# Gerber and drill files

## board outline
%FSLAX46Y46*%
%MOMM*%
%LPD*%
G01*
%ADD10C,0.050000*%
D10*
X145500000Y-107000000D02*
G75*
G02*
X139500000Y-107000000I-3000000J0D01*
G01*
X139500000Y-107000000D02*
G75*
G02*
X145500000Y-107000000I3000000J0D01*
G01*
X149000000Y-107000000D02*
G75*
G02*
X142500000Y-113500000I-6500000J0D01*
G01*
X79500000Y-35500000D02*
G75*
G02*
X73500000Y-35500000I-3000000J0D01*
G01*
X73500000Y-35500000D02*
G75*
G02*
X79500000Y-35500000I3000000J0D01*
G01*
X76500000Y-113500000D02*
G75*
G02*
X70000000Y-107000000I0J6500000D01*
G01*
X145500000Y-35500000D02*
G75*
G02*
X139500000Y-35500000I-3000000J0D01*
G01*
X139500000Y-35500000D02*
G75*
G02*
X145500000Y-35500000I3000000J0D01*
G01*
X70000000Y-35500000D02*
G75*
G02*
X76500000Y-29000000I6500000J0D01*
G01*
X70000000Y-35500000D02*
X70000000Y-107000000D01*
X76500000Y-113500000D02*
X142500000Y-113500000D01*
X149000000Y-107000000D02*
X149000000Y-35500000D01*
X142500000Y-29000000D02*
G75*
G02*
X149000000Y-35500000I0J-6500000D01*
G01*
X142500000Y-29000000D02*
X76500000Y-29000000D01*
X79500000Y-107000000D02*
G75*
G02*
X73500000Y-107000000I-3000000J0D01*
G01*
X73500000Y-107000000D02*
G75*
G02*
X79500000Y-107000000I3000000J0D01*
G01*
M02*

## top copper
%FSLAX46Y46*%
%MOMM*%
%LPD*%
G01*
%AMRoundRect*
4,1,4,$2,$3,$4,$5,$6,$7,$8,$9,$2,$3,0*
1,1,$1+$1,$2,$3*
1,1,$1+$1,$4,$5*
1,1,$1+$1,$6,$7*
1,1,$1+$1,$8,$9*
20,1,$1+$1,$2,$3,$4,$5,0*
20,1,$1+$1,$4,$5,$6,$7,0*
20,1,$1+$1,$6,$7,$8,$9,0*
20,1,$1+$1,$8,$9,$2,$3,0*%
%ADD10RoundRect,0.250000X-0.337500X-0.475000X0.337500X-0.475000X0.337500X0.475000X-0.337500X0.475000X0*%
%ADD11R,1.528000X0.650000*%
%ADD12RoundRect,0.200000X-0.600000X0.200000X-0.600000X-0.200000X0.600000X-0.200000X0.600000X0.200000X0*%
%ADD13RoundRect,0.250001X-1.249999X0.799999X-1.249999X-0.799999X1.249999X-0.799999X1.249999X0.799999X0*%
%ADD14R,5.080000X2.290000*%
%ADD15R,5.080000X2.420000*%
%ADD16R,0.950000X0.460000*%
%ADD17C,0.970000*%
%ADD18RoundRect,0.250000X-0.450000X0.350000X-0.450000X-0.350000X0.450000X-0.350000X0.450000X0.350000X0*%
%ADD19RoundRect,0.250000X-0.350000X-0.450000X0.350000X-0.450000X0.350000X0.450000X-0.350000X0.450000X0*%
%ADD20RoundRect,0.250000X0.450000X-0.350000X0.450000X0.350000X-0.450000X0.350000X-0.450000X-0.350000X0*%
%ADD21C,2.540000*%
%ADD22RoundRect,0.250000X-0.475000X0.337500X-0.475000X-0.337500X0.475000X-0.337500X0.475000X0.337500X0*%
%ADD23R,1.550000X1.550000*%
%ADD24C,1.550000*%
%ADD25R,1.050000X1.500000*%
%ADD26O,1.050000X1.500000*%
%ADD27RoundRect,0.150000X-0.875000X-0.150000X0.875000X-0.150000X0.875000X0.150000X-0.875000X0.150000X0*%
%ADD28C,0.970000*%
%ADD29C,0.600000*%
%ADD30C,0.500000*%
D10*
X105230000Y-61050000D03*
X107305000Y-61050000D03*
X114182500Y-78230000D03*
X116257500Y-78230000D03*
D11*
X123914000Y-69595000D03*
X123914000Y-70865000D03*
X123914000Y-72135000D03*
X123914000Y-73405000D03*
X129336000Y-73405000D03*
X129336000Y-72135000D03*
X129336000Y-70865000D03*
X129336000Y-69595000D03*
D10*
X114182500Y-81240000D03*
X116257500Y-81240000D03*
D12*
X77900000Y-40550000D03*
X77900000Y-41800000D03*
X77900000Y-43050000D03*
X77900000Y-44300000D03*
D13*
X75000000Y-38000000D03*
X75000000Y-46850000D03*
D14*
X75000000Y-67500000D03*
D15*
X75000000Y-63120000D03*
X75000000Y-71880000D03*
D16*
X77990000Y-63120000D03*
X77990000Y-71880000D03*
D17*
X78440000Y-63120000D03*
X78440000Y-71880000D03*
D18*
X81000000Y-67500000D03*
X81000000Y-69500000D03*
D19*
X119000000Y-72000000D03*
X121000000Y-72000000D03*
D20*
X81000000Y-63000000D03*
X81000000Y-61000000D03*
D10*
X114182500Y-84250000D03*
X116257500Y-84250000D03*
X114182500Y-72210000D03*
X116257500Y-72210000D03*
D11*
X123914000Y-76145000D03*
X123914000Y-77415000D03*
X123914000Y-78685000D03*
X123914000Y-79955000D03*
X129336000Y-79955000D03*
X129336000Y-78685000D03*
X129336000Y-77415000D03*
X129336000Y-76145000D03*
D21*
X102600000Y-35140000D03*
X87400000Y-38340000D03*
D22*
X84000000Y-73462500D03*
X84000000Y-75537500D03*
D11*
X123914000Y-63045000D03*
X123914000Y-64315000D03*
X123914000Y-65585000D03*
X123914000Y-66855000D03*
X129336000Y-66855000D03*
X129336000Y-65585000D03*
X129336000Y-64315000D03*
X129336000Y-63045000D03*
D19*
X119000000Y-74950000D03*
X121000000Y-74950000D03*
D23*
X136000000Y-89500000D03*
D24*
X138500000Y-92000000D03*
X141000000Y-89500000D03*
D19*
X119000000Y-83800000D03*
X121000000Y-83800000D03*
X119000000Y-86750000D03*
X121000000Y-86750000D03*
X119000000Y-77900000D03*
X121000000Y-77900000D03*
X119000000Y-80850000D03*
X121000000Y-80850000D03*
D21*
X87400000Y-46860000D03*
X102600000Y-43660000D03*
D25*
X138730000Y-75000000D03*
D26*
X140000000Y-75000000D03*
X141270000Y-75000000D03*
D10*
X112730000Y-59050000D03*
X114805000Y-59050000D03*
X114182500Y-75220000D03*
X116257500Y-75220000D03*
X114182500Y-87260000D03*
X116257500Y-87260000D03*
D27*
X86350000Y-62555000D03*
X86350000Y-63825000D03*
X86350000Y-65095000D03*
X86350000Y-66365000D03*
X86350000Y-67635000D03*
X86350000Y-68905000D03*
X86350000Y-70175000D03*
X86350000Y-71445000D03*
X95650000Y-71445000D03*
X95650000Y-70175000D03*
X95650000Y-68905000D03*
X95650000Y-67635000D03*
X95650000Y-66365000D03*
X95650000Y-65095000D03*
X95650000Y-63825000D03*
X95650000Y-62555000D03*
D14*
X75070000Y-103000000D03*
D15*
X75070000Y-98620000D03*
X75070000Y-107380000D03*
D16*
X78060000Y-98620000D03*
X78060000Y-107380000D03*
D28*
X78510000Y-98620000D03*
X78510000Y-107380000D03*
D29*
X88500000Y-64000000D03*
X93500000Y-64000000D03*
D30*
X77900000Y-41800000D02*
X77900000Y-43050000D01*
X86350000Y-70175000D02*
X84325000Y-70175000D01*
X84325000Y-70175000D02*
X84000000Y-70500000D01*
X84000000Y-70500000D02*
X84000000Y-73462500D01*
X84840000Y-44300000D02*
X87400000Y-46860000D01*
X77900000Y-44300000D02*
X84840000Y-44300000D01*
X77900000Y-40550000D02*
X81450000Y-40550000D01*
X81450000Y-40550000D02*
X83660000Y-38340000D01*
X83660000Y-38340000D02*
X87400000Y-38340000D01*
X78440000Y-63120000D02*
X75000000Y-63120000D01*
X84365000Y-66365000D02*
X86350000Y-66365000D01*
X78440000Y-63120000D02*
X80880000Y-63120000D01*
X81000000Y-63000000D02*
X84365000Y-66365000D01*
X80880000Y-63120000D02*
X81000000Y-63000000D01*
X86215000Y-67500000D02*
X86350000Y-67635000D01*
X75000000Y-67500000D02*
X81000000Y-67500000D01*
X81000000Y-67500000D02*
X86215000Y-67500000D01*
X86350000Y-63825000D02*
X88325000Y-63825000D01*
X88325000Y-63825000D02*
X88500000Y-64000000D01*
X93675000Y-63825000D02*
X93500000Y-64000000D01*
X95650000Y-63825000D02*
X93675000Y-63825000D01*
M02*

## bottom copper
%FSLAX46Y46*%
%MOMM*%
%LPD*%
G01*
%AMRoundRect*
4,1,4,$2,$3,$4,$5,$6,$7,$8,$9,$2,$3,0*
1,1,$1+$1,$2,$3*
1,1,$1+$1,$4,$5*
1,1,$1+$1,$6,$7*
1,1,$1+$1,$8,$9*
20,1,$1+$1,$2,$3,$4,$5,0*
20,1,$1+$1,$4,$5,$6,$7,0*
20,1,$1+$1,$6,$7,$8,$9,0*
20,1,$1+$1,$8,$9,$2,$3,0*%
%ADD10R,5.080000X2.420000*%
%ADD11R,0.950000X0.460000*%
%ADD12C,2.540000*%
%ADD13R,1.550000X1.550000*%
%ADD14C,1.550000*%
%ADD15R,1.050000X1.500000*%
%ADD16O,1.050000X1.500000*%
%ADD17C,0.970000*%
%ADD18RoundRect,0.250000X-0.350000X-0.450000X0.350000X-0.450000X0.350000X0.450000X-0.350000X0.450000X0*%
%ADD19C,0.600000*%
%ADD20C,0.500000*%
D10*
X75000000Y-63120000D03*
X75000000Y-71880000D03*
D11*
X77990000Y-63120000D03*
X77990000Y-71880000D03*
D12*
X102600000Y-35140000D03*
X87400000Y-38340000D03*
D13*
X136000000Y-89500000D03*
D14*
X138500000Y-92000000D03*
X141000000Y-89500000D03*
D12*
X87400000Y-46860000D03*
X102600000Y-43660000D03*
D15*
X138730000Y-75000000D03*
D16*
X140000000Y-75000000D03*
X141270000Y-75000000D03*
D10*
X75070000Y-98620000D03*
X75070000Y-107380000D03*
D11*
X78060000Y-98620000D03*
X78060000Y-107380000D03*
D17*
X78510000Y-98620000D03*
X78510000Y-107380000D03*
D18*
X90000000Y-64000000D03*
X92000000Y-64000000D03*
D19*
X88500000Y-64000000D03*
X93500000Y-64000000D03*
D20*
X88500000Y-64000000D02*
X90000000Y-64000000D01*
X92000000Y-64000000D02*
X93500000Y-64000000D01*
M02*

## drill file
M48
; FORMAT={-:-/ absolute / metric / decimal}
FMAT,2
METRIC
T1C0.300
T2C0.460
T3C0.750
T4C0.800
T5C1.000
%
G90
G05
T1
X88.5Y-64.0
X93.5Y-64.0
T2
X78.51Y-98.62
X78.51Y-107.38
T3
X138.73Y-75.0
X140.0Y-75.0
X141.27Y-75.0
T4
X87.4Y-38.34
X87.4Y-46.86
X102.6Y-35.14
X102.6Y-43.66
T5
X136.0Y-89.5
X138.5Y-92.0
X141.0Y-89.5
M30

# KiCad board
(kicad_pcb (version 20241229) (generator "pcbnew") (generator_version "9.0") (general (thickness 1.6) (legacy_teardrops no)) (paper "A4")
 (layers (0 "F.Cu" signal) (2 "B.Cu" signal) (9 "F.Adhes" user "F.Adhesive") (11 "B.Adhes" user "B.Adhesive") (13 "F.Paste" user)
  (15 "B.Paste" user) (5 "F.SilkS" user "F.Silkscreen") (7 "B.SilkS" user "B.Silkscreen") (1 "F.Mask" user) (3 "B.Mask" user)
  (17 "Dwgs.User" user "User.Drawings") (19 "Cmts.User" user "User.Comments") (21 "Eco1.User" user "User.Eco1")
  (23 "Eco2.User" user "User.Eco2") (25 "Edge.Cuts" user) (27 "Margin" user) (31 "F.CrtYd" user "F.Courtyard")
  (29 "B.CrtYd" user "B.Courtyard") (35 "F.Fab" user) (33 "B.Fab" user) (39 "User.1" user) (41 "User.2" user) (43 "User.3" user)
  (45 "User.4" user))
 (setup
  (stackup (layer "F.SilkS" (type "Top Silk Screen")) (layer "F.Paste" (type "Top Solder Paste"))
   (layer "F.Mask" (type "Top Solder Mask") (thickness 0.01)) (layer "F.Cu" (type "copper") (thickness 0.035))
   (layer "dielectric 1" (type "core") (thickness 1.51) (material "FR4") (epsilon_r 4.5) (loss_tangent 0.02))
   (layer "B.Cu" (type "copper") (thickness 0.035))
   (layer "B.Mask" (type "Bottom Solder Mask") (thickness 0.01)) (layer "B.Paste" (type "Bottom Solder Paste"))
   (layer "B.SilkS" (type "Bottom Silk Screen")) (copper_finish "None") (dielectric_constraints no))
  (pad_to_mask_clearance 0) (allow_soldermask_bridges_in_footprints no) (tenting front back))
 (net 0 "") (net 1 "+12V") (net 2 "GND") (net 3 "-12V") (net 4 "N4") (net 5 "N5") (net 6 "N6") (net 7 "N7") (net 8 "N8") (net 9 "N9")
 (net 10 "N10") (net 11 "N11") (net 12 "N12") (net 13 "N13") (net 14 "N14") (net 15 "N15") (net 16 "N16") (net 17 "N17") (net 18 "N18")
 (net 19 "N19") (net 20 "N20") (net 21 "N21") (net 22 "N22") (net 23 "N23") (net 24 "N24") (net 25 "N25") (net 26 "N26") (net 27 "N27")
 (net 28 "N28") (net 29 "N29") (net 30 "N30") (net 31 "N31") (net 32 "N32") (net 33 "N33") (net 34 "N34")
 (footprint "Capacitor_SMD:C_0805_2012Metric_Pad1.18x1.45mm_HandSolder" (layer "F.Cu") (at 106.2675 61.05)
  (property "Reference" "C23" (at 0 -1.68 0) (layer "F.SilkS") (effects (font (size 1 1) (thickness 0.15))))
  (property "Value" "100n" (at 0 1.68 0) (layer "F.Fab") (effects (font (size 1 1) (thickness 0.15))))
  (pad "1" smd roundrect (at -1.0375 0) (size 1.175 1.45) (layers "F.Cu" "F.Mask" "F.Paste") (roundrect_rratio 0.212766) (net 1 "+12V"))
  (pad "2" smd roundrect (at 1.0375 0) (size 1.175 1.45) (layers "F.Cu" "F.Mask" "F.Paste") (roundrect_rratio 0.212766) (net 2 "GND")))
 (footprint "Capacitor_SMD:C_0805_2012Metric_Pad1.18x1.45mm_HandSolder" (layer "F.Cu") (at 115.22 78.23)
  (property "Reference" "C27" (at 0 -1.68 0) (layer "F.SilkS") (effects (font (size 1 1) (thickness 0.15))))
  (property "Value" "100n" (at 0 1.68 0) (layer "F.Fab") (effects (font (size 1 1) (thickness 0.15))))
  (pad "1" smd roundrect (at -1.0375 0) (size 1.175 1.45) (layers "F.Cu" "F.Mask" "F.Paste") (roundrect_rratio 0.212766) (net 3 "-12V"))
  (pad "2" smd roundrect (at 1.0375 0) (size 1.175 1.45) (layers "F.Cu" "F.Mask" "F.Paste") (roundrect_rratio 0.212766) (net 2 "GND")))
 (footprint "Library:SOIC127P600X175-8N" (layer "F.Cu") (at 126.625 71.5)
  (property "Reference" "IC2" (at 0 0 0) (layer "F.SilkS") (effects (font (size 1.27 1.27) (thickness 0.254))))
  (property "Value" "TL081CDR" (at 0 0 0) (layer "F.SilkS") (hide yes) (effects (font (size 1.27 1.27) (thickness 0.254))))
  (pad "1" smd rect (at -2.711 -1.905 90) (size 0.65 1.528) (layers "F.Cu" "F.Mask" "F.Paste") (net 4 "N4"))
  (pad "2" smd rect (at -2.711 -0.635 90) (size 0.65 1.528) (layers "F.Cu" "F.Mask" "F.Paste") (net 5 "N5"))
  (pad "3" smd rect (at -2.711 0.635 90) (size 0.65 1.528) (layers "F.Cu" "F.Mask" "F.Paste") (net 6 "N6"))
  (pad "4" smd rect (at -2.711 1.905 90) (size 0.65 1.528) (layers "F.Cu" "F.Mask" "F.Paste") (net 3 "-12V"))
  (pad "5" smd rect (at 2.711 1.905 90) (size 0.65 1.528) (layers "F.Cu" "F.Mask" "F.Paste") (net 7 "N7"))
  (pad "6" smd rect (at 2.711 0.635 90) (size 0.65 1.528) (layers "F.Cu" "F.Mask" "F.Paste") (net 5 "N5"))
  (pad "7" smd rect (at 2.711 -0.635 90) (size 0.65 1.528) (layers "F.Cu" "F.Mask" "F.Paste") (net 1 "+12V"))
  (pad "8" smd rect (at 2.711 -1.905 90) (size 0.65 1.528) (layers "F.Cu" "F.Mask" "F.Paste") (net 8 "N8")))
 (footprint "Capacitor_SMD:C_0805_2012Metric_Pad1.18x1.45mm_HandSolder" (layer "F.Cu") (at 115.22 81.24)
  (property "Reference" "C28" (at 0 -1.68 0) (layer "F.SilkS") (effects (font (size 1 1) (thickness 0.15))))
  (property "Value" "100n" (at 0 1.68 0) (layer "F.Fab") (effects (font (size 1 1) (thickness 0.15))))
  (pad "1" smd roundrect (at -1.0375 0) (size 1.175 1.45) (layers "F.Cu" "F.Mask" "F.Paste") (roundrect_rratio 0.212766) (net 1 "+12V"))
  (pad "2" smd roundrect (at 1.0375 0) (size 1.175 1.45) (layers "F.Cu" "F.Mask" "F.Paste") (roundrect_rratio 0.212766) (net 2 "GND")))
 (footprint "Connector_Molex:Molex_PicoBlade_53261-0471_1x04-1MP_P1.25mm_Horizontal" (layer "F.Cu") (at 75.5 42.425 -90)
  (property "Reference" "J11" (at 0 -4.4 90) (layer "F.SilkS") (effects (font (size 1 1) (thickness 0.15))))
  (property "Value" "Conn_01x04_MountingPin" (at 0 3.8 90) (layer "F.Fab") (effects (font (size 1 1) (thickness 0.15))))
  (pad "1" smd roundrect (at -1.875 -2.4 270) (size 0.8 1.6) (layers "F.Cu" "F.Mask" "F.Paste") (roundrect_rratio 0.25) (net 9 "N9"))
  (pad "2" smd roundrect (at -0.625 -2.4 270) (size 0.8 1.6) (layers "F.Cu" "F.Mask" "F.Paste") (roundrect_rratio 0.25) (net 2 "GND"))
  (pad "3" smd roundrect (at 0.625 -2.4 270) (size 0.8 1.6) (layers "F.Cu" "F.Mask" "F.Paste") (roundrect_rratio 0.25) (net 2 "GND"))
  (pad "4" smd roundrect (at 1.875 -2.4 270) (size 0.8 1.6) (layers "F.Cu" "F.Mask" "F.Paste") (roundrect_rratio 0.25) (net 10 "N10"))
  (pad "MP" smd roundrect (at -4.425 0.5 270) (size 2.1 3) (layers "F.Cu" "F.Mask" "F.Paste") (roundrect_rratio 0.119048) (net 2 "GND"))
  (pad "MP" smd roundrect (at 4.425 0.5 270) (size 2.1 3) (layers "F.Cu" "F.Mask" "F.Paste") (roundrect_rratio 0.119048) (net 2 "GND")))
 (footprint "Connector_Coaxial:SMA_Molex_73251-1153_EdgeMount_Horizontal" (layer "F.Cu") (at 76.72 67.5)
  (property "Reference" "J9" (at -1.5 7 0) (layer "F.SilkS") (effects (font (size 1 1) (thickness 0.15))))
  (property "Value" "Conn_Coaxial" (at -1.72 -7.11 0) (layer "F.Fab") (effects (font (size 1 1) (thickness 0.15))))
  (pad "1" smd rect (at -1.72 0) (size 5.08 2.29) (layers "F.Cu" "F.Mask" "F.Paste") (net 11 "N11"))
  (pad "2" smd rect (at -1.72 -4.38) (size 5.08 2.42) (layers "F.Cu" "F.Mask" "F.Paste") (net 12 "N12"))
  (pad "2" smd rect (at -1.72 -4.38) (size 5.08 2.42) (layers "B.Cu" "B.Mask" "B.Paste") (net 12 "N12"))
  (pad "2" smd rect (at -1.72 4.38) (size 5.08 2.42) (layers "F.Cu" "F.Mask" "F.Paste") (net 12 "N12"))
  (pad "2" smd rect (at -1.72 4.38) (size 5.08 2.42) (layers "B.Cu" "B.Mask" "B.Paste") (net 12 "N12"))
  (pad "2" smd rect (at 1.27 -4.38) (size 0.95 0.46) (layers "F.Cu") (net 12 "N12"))
  (pad "2" smd rect (at 1.27 -4.38) (size 0.95 0.46) (layers "B.Cu") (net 12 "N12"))
  (pad "2" smd rect (at 1.27 4.38) (size 0.95 0.46) (layers "F.Cu") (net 12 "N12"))
  (pad "2" smd rect (at 1.27 4.38) (size 0.95 0.46) (layers "B.Cu") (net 12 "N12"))
  (pad "2" smd circle (at 1.72 -4.38) (size 0.97 0.97) (layers "F.Cu" "F.Mask" "F.Paste") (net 12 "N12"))
  (pad "2" smd circle (at 1.72 4.38) (size 0.97 0.97) (layers "F.Cu" "F.Mask" "F.Paste") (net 12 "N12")))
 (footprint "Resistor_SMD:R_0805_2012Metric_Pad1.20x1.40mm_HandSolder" (layer "F.Cu") (at 81 68.5 -90)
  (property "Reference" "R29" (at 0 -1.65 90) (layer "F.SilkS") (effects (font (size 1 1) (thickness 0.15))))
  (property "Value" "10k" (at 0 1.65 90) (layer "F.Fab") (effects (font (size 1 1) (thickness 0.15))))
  (pad "1" smd roundrect (at -1 0 270) (size 1.2 1.4) (layers "F.Cu" "F.Mask" "F.Paste") (roundrect_rratio 0.208333) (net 11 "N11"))
  (pad "2" smd roundrect (at 1 0 270) (size 1.2 1.4) (layers "F.Cu" "F.Mask" "F.Paste") (roundrect_rratio 0.208333) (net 2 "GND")))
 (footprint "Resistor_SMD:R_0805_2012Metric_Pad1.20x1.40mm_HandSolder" (layer "F.Cu") (at 120 72)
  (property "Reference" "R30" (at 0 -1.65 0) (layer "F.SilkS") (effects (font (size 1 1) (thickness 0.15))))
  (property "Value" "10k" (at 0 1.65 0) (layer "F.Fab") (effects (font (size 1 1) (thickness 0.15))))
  (pad "1" smd roundrect (at -1 0) (size 1.2 1.4) (layers "F.Cu" "F.Mask" "F.Paste") (roundrect_rratio 0.208333) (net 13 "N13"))
  (pad "2" smd roundrect (at 1 0) (size 1.2 1.4) (layers "F.Cu" "F.Mask" "F.Paste") (roundrect_rratio 0.208333) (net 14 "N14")))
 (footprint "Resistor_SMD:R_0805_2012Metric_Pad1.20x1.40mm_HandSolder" (layer "F.Cu") (at 81 62 90)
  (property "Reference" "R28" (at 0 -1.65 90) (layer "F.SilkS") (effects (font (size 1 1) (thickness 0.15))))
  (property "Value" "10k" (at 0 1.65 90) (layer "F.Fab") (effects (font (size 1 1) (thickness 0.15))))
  (pad "1" smd roundrect (at -1 0 90) (size 1.2 1.4) (layers "F.Cu" "F.Mask" "F.Paste") (roundrect_rratio 0.208333) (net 12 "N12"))
  (pad "2" smd roundrect (at 1 0 90) (size 1.2 1.4) (layers "F.Cu" "F.Mask" "F.Paste") (roundrect_rratio 0.208333) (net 2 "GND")))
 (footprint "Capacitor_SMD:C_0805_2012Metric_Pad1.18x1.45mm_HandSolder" (layer "F.Cu") (at 115.22 84.25)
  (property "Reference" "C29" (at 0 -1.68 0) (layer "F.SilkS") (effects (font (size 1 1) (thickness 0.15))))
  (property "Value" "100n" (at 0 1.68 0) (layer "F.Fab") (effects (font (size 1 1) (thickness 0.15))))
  (pad "1" smd roundrect (at -1.0375 0) (size 1.175 1.45) (layers "F.Cu" "F.Mask" "F.Paste") (roundrect_rratio 0.212766) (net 3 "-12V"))
  (pad "2" smd roundrect (at 1.0375 0) (size 1.175 1.45) (layers "F.Cu" "F.Mask" "F.Paste") (roundrect_rratio 0.212766) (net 2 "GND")))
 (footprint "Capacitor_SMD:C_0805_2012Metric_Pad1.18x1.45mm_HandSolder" (layer "F.Cu") (at 115.22 72.21)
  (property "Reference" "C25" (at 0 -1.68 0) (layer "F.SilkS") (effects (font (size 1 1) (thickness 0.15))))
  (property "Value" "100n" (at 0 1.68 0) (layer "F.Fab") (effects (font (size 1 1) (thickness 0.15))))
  (pad "1" smd roundrect (at -1.0375 0) (size 1.175 1.45) (layers "F.Cu" "F.Mask" "F.Paste") (roundrect_rratio 0.212766) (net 3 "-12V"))
  (pad "2" smd roundrect (at 1.0375 0) (size 1.175 1.45) (layers "F.Cu" "F.Mask" "F.Paste") (roundrect_rratio 0.212766) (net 2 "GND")))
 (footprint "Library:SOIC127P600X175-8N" (layer "F.Cu") (at 126.625 78.05)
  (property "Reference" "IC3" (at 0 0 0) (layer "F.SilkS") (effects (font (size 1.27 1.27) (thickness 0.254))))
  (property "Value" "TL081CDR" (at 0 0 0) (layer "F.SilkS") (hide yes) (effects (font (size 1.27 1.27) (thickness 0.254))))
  (pad "1" smd rect (at -2.711 -1.905 90) (size 0.65 1.528) (layers "F.Cu" "F.Mask" "F.Paste") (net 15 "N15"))
  (pad "2" smd rect (at -2.711 -0.635 90) (size 0.65 1.528) (layers "F.Cu" "F.Mask" "F.Paste") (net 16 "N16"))
  (pad "3" smd rect (at -2.711 0.635 90) (size 0.65 1.528) (layers "F.Cu" "F.Mask" "F.Paste") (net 14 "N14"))
  (pad "4" smd rect (at -2.711 1.905 90) (size 0.65 1.528) (layers "F.Cu" "F.Mask" "F.Paste") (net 3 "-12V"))
  (pad "5" smd rect (at 2.711 1.905 90) (size 0.65 1.528) (layers "F.Cu" "F.Mask" "F.Paste") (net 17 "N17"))
  (pad "6" smd rect (at 2.711 0.635 90) (size 0.65 1.528) (layers "F.Cu" "F.Mask" "F.Paste") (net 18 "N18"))
  (pad "7" smd rect (at 2.711 -0.635 90) (size 0.65 1.528) (layers "F.Cu" "F.Mask" "F.Paste") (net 1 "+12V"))
  (pad "8" smd rect (at 2.711 -1.905 90) (size 0.65 1.528) (layers "F.Cu" "F.Mask" "F.Paste") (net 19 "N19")))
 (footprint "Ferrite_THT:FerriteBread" (layer "F.Cu") (at 95.1 32.64 180)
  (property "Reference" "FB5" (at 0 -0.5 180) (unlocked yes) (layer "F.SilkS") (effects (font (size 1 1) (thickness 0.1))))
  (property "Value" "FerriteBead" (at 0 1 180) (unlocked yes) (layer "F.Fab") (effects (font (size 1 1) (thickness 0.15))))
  (pad "1" thru_hole circle (at -7.5 -2.5 180) (size 2.54 2.54) (drill 0.8) (layers "*.Cu" "*.Mask") (remove_unused_layers no)
   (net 1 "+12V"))
  (pad "2" thru_hole circle (at 7.7 -5.7 180) (size 2.54 2.54) (drill 0.8) (layers "*.Cu" "*.Mask") (remove_unused_layers no) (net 9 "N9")))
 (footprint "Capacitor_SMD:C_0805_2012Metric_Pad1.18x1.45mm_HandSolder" (layer "F.Cu") (at 84 74.5 -90)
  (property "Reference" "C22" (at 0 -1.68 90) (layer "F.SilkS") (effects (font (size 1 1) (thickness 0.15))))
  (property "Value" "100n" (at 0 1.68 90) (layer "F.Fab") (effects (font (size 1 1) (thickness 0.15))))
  (pad "1" smd roundrect (at -1.0375 0 270) (size 1.175 1.45) (layers "F.Cu" "F.Mask" "F.Paste") (roundrect_rratio 0.212766) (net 3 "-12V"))
  (pad "2" smd roundrect (at 1.0375 0 270) (size 1.175 1.45) (layers "F.Cu" "F.Mask" "F.Paste") (roundrect_rratio 0.212766) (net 2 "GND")))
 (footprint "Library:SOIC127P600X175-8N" (layer "F.Cu") (at 126.625 64.95)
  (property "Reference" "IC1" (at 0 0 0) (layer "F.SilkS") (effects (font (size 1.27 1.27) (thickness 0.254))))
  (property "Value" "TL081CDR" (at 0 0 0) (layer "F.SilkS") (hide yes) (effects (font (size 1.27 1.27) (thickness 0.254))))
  (pad "1" smd rect (at -2.711 -1.905 90) (size 0.65 1.528) (layers "F.Cu" "F.Mask" "F.Paste") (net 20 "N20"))
  (pad "2" smd rect (at -2.711 -0.635 90) (size 0.65 1.528) (layers "F.Cu" "F.Mask" "F.Paste") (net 13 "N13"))
  (pad "3" smd rect (at -2.711 0.635 90) (size 0.65 1.528) (layers "F.Cu" "F.Mask" "F.Paste") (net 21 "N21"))
  (pad "4" smd rect (at -2.711 1.905 90) (size 0.65 1.528) (layers "F.Cu" "F.Mask" "F.Paste") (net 3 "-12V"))
  (pad "5" smd rect (at 2.711 1.905 90) (size 0.65 1.528) (layers "F.Cu" "F.Mask" "F.Paste") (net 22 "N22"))
  (pad "6" smd rect (at 2.711 0.635 90) (size 0.65 1.528) (layers "F.Cu" "F.Mask" "F.Paste") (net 13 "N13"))
  (pad "7" smd rect (at 2.711 -0.635 90) (size 0.65 1.528) (layers "F.Cu" "F.Mask" "F.Paste") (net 1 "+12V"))
  (pad "8" smd rect (at 2.711 -1.905 90) (size 0.65 1.528) (layers "F.Cu" "F.Mask" "F.Paste") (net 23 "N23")))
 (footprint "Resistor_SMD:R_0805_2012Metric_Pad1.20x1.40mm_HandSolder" (layer "F.Cu") (at 120 74.95)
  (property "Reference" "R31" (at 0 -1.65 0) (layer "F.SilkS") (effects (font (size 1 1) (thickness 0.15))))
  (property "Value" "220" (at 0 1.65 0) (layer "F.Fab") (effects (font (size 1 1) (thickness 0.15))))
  (pad "1" smd roundrect (at -1 0) (size 1.2 1.4) (layers "F.Cu" "F.Mask" "F.Paste") (roundrect_rratio 0.208333) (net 1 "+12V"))
  (pad "2" smd roundrect (at 1 0) (size 1.2 1.4) (layers "F.Cu" "F.Mask" "F.Paste") (roundrect_rratio 0.208333) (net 6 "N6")))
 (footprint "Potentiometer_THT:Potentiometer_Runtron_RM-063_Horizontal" (layer "F.Cu") (at 136 89.5)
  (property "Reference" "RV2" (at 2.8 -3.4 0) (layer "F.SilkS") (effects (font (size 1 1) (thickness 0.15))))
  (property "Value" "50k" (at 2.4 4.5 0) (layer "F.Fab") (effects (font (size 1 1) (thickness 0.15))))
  (pad "1" thru_hole rect (at 0 0) (size 1.55 1.55) (drill 1) (layers "*.Cu" "*.Mask") (remove_unused_layers no) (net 6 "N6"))
  (pad "2" thru_hole circle (at 2.5 2.5) (size 1.55 1.55) (drill 1) (layers "*.Cu" "*.Mask") (remove_unused_layers no) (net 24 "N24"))
  (pad "3" thru_hole circle (at 5 0) (size 1.55 1.55) (drill 1) (layers "*.Cu" "*.Mask") (remove_unused_layers no) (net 2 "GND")))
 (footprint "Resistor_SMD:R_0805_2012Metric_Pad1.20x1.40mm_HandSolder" (layer "F.Cu") (at 120 83.8)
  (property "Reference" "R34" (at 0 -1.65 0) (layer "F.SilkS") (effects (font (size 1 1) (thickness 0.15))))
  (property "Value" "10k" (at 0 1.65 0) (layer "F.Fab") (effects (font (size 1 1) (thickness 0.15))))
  (pad "1" smd roundrect (at -1 0) (size 1.2 1.4) (layers "F.Cu" "F.Mask" "F.Paste") (roundrect_rratio 0.208333) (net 2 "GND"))
  (pad "2" smd roundrect (at 1 0) (size 1.2 1.4) (layers "F.Cu" "F.Mask" "F.Paste") (roundrect_rratio 0.208333) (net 16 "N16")))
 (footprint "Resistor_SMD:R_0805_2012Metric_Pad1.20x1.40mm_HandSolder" (layer "F.Cu") (at 120 86.75)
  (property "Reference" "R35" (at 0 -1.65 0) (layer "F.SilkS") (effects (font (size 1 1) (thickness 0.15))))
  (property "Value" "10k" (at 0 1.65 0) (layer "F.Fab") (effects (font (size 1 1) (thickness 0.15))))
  (pad "1" smd roundrect (at -1 0) (size 1.2 1.4) (layers "F.Cu" "F.Mask" "F.Paste") (roundrect_rratio 0.208333) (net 16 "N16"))
  (pad "2" smd roundrect (at 1 0) (size 1.2 1.4) (layers "F.Cu" "F.Mask" "F.Paste") (roundrect_rratio 0.208333) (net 18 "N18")))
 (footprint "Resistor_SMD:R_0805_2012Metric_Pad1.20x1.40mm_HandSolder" (layer "F.Cu") (at 120 77.9)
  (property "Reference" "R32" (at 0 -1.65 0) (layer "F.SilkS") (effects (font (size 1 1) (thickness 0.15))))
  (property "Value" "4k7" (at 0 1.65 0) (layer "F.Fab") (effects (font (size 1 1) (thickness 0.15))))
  (pad "1" smd roundrect (at -1 0) (size 1.2 1.4) (layers "F.Cu" "F.Mask" "F.Paste") (roundrect_rratio 0.208333) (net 6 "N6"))
  (pad "2" smd roundrect (at 1 0) (size 1.2 1.4) (layers "F.Cu" "F.Mask" "F.Paste") (roundrect_rratio 0.208333) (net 2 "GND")))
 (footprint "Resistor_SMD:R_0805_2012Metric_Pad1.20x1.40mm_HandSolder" (layer "F.Cu") (at 120 80.85)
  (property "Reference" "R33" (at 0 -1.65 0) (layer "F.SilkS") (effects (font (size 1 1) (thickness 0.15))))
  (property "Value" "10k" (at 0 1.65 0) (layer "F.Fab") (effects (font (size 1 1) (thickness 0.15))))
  (pad "1" smd roundrect (at -1 0) (size 1.2 1.4) (layers "F.Cu" "F.Mask" "F.Paste") (roundrect_rratio 0.208333) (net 5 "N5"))
  (pad "2" smd roundrect (at 1 0) (size 1.2 1.4) (layers "F.Cu" "F.Mask" "F.Paste") (roundrect_rratio 0.208333) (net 14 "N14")))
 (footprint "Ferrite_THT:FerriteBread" (layer "F.Cu") (at 94.9 49.36)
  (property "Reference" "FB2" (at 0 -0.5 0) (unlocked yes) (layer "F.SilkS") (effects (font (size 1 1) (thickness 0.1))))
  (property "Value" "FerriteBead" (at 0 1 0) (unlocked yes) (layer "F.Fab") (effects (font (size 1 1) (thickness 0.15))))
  (pad "1" thru_hole circle (at -7.5 -2.5) (size 2.54 2.54) (drill 0.8) (layers "*.Cu" "*.Mask") (remove_unused_layers no) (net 10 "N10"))
  (pad "2" thru_hole circle (at 7.7 -5.7) (size 2.54 2.54) (drill 0.8) (layers "*.Cu" "*.Mask") (remove_unused_layers no) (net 3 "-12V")))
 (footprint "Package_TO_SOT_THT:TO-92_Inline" (layer "F.Cu") (at 138.73 75)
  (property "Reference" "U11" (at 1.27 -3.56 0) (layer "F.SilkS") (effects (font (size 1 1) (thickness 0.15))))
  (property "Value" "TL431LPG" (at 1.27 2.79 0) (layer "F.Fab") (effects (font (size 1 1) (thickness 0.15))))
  (pad "1" thru_hole rect (at 0 0) (size 1.05 1.5) (drill 0.75) (layers "*.Cu" "*.Mask") (remove_unused_layers no) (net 24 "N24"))
  (pad "2" thru_hole oval (at 1.27 0) (size 1.05 1.5) (drill 0.75) (layers "*.Cu" "*.Mask") (remove_unused_layers no) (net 2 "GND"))
  (pad "3" thru_hole oval (at 2.54 0) (size 1.05 1.5) (drill 0.75) (layers "*.Cu" "*.Mask") (remove_unused_layers no) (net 6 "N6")))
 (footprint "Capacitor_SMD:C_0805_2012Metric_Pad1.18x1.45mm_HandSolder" (layer "F.Cu") (at 113.7675 59.05)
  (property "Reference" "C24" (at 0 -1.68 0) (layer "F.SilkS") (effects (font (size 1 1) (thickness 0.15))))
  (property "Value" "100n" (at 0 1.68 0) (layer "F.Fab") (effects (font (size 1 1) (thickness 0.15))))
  (pad "1" smd roundrect (at -1.0375 0) (size 1.175 1.45) (layers "F.Cu" "F.Mask" "F.Paste") (roundrect_rratio 0.212766) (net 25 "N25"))
  (pad "2" smd roundrect (at 1.0375 0) (size 1.175 1.45) (layers "F.Cu" "F.Mask" "F.Paste") (roundrect_rratio 0.212766) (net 21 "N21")))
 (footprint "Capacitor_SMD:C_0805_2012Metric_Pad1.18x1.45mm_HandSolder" (layer "F.Cu") (at 115.22 75.22)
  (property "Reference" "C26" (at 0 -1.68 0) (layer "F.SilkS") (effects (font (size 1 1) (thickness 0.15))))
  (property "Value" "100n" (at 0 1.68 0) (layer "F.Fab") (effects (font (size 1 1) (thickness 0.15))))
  (pad "1" smd roundrect (at -1.0375 0) (size 1.175 1.45) (layers "F.Cu" "F.Mask" "F.Paste") (roundrect_rratio 0.212766) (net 1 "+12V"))
  (pad "2" smd roundrect (at 1.0375 0) (size 1.175 1.45) (layers "F.Cu" "F.Mask" "F.Paste") (roundrect_rratio 0.212766) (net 2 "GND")))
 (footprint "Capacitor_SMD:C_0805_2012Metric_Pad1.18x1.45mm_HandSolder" (layer "F.Cu") (at 115.22 87.26)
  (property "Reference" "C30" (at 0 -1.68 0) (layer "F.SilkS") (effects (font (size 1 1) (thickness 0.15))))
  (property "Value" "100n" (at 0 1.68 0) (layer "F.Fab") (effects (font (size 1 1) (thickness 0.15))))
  (pad "1" smd roundrect (at -1.0375 0) (size 1.175 1.45) (layers "F.Cu" "F.Mask" "F.Paste") (roundrect_rratio 0.212766) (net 1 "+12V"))
  (pad "2" smd roundrect (at 1.0375 0) (size 1.175 1.45) (layers "F.Cu" "F.Mask" "F.Paste") (roundrect_rratio 0.212766) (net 2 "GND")))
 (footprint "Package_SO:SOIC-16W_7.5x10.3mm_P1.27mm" (layer "F.Cu") (at 91 67)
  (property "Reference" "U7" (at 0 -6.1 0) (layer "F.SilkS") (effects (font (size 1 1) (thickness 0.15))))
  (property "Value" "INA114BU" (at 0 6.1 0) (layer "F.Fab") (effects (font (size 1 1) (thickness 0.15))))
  (pad "1" smd roundrect (at -4.65 -4.445) (size 2.05 0.6) (layers "F.Cu" "F.Mask" "F.Paste") (roundrect_rratio 0.25) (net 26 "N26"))
  (pad "2" smd roundrect (at -4.65 -3.175) (size 2.05 0.6) (layers "F.Cu" "F.Mask" "F.Paste") (roundrect_rratio 0.25) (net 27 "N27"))
  (pad "3" smd roundrect (at -4.65 -1.905) (size 2.05 0.6) (layers "F.Cu" "F.Mask" "F.Paste") (roundrect_rratio 0.25) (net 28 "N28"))
  (pad "4" smd roundrect (at -4.65 -0.635) (size 2.05 0.6) (layers "F.Cu" "F.Mask" "F.Paste") (roundrect_rratio 0.25) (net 12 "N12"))
  (pad "5" smd roundrect (at -4.65 0.635) (size 2.05 0.6) (layers "F.Cu" "F.Mask" "F.Paste") (roundrect_rratio 0.25) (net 11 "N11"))
  (pad "6" smd roundrect (at -4.65 1.905) (size 2.05 0.6) (layers "F.Cu" "F.Mask" "F.Paste") (roundrect_rratio 0.25) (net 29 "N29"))
  (pad "7" smd roundrect (at -4.65 3.175) (size 2.05 0.6) (layers "F.Cu" "F.Mask" "F.Paste") (roundrect_rratio 0.25) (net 3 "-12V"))
  (pad "8" smd roundrect (at -4.65 4.445) (size 2.05 0.6) (layers "F.Cu" "F.Mask" "F.Paste") (roundrect_rratio 0.25) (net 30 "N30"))
  (pad "9" smd roundrect (at 4.65 4.445) (size 2.05 0.6) (layers "F.Cu" "F.Mask" "F.Paste") (roundrect_rratio 0.25) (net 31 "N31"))
  (pad "10" smd roundrect (at 4.65 3.175) (size 2.05 0.6) (layers "F.Cu" "F.Mask" "F.Paste") (roundrect_rratio 0.25) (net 2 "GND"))
  (pad "11" smd roundrect (at 4.65 1.905) (size 2.05 0.6) (layers "F.Cu" "F.Mask" "F.Paste") (roundrect_rratio 0.25) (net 25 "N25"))
  (pad "12" smd roundrect (at 4.65 0.635) (size 2.05 0.6) (layers "F.Cu" "F.Mask" "F.Paste") (roundrect_rratio 0.25) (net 25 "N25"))
  (pad "13" smd roundrect (at 4.65 -0.635) (size 2.05 0.6) (layers "F.Cu" "F.Mask" "F.Paste") (roundrect_rratio 0.25) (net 1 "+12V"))
  (pad "14" smd roundrect (at 4.65 -1.905) (size 2.05 0.6) (layers "F.Cu" "F.Mask" "F.Paste") (roundrect_rratio 0.25) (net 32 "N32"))
  (pad "15" smd roundrect (at 4.65 -3.175) (size 2.05 0.6) (layers "F.Cu" "F.Mask" "F.Paste") (roundrect_rratio 0.25) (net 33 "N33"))
  (pad "16" smd roundrect (at 4.65 -4.445) (size 2.05 0.6) (layers "F.Cu" "F.Mask" "F.Paste") (roundrect_rratio 0.25) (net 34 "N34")))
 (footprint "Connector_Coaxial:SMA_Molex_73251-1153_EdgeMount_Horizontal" (layer "F.Cu") (at 76.79 103)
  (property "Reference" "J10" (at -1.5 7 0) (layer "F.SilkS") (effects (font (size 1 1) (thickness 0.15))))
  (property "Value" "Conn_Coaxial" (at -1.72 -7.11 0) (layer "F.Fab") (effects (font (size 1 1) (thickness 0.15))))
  (pad "1" smd rect (at -1.72 0) (size 5.08 2.29) (layers "F.Cu" "F.Mask" "F.Paste") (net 18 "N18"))
  (pad "2" smd rect (at -1.72 -4.38) (size 5.08 2.42) (layers "F.Cu" "F.Mask" "F.Paste") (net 2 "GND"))
  (pad "2" smd rect (at -1.72 -4.38) (size 5.08 2.42) (layers "B.Cu" "B.Mask" "B.Paste") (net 2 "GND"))
  (pad "2" smd rect (at -1.72 4.38) (size 5.08 2.42) (layers "F.Cu" "F.Mask" "F.Paste") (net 2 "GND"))
  (pad "2" smd rect (at -1.72 4.38) (size 5.08 2.42) (layers "B.Cu" "B.Mask" "B.Paste") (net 2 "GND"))
  (pad "2" smd rect (at 1.27 -4.38) (size 0.95 0.46) (layers "F.Cu") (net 2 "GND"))
  (pad "2" smd rect (at 1.27 -4.38) (size 0.95 0.46) (layers "B.Cu") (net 2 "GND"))
  (pad "2" smd rect (at 1.27 4.38) (size 0.95 0.46) (layers "F.Cu") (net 2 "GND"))
  (pad "2" smd rect (at 1.27 4.38) (size 0.95 0.46) (layers "B.Cu") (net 2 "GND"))
  (pad "2" thru_hole circle (at 1.72 -4.38) (size 0.97 0.97) (drill 0.46) (layers "*.Cu") (remove_unused_layers no) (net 2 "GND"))
  (pad "2" thru_hole circle (at 1.72 4.38) (size 0.97 0.97) (drill 0.46) (layers "*.Cu") (remove_unused_layers no) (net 2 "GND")))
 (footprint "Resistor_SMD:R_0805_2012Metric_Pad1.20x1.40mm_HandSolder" (layer "B.Cu") (at 91 64)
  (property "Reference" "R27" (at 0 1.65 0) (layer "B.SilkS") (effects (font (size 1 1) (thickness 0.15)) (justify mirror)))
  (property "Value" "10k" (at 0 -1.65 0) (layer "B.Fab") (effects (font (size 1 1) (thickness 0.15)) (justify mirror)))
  (pad "1" smd roundrect (at -1 0) (size 1.2 1.4) (layers "B.Cu" "B.Mask" "B.Paste") (roundrect_rratio 0.208333) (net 27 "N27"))
  (pad "2" smd roundrect (at 1 0) (size 1.2 1.4) (layers "B.Cu" "B.Mask" "B.Paste") (roundrect_rratio 0.208333) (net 33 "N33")))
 (gr_circle (center 142.5 107) (end 142.5 104) (stroke (width 0.05) (type default)) (fill no) (layer "Edge.Cuts"))
 (gr_arc (start 149 107) (mid 147.096194 111.596194) (end 142.5 113.5) (stroke (width 0.05) (type default)) (layer "Edge.Cuts"))
 (gr_circle (center 76.5 35.5) (end 76.5 32.5) (stroke (width 0.05) (type default)) (fill no) (layer "Edge.Cuts"))
 (gr_arc (start 76.5 113.5) (mid 71.903806 111.596194) (end 70 107) (stroke (width 0.05) (type default)) (layer "Edge.Cuts"))
 (gr_circle (center 142.5 35.5) (end 142.5 32.5) (stroke (width 0.05) (type default)) (fill no) (layer "Edge.Cuts"))
 (gr_arc (start 70 35.5) (mid 71.903806 30.903806) (end 76.5 29) (stroke (width 0.05) (type default)) (layer "Edge.Cuts"))
 (gr_line (start 70 35.5) (end 70 107) (stroke (width 0.05) (type default)) (layer "Edge.Cuts"))
 (gr_line (start 76.5 113.5) (end 142.5 113.5) (stroke (width 0.05) (type default)) (layer "Edge.Cuts"))
 (gr_line (start 149 107) (end 149 35.5) (stroke (width 0.05) (type default)) (layer "Edge.Cuts"))
 (gr_arc (start 142.5 29) (mid 147.096194 30.903806) (end 149 35.5) (stroke (width 0.05) (type default)) (layer "Edge.Cuts"))
 (gr_line (start 142.5 29) (end 76.5 29) (stroke (width 0.05) (type default)) (layer "Edge.Cuts"))
 (gr_circle (center 76.5 107) (end 76.5 104) (stroke (width 0.05) (type default)) (fill no) (layer "Edge.Cuts"))
 (segment (start 77.9 41.8) (end 77.9 43.05) (width 0.5) (layer "F.Cu") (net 2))
 (segment (start 86.35 70.175) (end 84.325 70.175) (width 0.5) (layer "F.Cu") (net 3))
 (segment (start 84.325 70.175) (end 84 70.5) (width 0.5) (layer "F.Cu") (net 3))
 (segment (start 84 70.5) (end 84 73.4625) (width 0.5) (layer "F.Cu") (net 3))
 (segment (start 84.84 44.3) (end 87.4 46.86) (width 0.5) (layer "F.Cu") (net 10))
 (segment (start 77.9 44.3) (end 84.84 44.3) (width 0.5) (layer "F.Cu") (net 10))
 (segment (start 77.9 40.55) (end 81.45 40.55) (width 0.5) (layer "F.Cu") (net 9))
 (segment (start 81.45 40.55) (end 83.66 38.34) (width 0.5) (layer "F.Cu") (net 9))
 (segment (start 83.66 38.34) (end 87.4 38.34) (width 0.5) (layer "F.Cu") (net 9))
 (segment (start 78.44 63.12) (end 75 63.12) (width 0.5) (layer "F.Cu") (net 12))
 (segment (start 84.365 66.365) (end 86.35 66.365) (width 0.5) (layer "F.Cu") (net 12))
 (segment (start 78.44 63.12) (end 80.88 63.12) (width 0.5) (layer "F.Cu") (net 12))
 (segment (start 81 63) (end 84.365 66.365) (width 0.5) (layer "F.Cu") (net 12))
 (segment (start 80.88 63.12) (end 81 63) (width 0.5) (layer "F.Cu") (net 12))
 (segment (start 86.215 67.5) (end 86.35 67.635) (width 0.5) (layer "F.Cu") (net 11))
 (segment (start 75 67.5) (end 81 67.5) (width 0.5) (layer "F.Cu") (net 11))
 (segment (start 81 67.5) (end 86.215 67.5) (width 0.5) (layer "F.Cu") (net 11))
 (segment (start 86.35 63.825) (end 88.325 63.825) (width 0.5) (layer "F.Cu") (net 27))
 (segment (start 88.325 63.825) (end 88.5 64) (width 0.5) (layer "F.Cu") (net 27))
 (via (at 88.5 64) (size 0.6) (drill 0.3) (layers "F.Cu" "B.Cu") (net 27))
 (segment (start 88.5 64) (end 90 64) (width 0.5) (layer "B.Cu") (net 27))
 (segment (start 93.675 63.825) (end 93.5 64) (width 0.5) (layer "F.Cu") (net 33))
 (segment (start 95.65 63.825) (end 93.675 63.825) (width 0.5) (layer "F.Cu") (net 33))
 (via (at 93.5 64) (size 0.6) (drill 0.3) (layers "F.Cu" "B.Cu") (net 33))
 (segment (start 92 64) (end 93.5 64) (width 0.5) (layer "B.Cu") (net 33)))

